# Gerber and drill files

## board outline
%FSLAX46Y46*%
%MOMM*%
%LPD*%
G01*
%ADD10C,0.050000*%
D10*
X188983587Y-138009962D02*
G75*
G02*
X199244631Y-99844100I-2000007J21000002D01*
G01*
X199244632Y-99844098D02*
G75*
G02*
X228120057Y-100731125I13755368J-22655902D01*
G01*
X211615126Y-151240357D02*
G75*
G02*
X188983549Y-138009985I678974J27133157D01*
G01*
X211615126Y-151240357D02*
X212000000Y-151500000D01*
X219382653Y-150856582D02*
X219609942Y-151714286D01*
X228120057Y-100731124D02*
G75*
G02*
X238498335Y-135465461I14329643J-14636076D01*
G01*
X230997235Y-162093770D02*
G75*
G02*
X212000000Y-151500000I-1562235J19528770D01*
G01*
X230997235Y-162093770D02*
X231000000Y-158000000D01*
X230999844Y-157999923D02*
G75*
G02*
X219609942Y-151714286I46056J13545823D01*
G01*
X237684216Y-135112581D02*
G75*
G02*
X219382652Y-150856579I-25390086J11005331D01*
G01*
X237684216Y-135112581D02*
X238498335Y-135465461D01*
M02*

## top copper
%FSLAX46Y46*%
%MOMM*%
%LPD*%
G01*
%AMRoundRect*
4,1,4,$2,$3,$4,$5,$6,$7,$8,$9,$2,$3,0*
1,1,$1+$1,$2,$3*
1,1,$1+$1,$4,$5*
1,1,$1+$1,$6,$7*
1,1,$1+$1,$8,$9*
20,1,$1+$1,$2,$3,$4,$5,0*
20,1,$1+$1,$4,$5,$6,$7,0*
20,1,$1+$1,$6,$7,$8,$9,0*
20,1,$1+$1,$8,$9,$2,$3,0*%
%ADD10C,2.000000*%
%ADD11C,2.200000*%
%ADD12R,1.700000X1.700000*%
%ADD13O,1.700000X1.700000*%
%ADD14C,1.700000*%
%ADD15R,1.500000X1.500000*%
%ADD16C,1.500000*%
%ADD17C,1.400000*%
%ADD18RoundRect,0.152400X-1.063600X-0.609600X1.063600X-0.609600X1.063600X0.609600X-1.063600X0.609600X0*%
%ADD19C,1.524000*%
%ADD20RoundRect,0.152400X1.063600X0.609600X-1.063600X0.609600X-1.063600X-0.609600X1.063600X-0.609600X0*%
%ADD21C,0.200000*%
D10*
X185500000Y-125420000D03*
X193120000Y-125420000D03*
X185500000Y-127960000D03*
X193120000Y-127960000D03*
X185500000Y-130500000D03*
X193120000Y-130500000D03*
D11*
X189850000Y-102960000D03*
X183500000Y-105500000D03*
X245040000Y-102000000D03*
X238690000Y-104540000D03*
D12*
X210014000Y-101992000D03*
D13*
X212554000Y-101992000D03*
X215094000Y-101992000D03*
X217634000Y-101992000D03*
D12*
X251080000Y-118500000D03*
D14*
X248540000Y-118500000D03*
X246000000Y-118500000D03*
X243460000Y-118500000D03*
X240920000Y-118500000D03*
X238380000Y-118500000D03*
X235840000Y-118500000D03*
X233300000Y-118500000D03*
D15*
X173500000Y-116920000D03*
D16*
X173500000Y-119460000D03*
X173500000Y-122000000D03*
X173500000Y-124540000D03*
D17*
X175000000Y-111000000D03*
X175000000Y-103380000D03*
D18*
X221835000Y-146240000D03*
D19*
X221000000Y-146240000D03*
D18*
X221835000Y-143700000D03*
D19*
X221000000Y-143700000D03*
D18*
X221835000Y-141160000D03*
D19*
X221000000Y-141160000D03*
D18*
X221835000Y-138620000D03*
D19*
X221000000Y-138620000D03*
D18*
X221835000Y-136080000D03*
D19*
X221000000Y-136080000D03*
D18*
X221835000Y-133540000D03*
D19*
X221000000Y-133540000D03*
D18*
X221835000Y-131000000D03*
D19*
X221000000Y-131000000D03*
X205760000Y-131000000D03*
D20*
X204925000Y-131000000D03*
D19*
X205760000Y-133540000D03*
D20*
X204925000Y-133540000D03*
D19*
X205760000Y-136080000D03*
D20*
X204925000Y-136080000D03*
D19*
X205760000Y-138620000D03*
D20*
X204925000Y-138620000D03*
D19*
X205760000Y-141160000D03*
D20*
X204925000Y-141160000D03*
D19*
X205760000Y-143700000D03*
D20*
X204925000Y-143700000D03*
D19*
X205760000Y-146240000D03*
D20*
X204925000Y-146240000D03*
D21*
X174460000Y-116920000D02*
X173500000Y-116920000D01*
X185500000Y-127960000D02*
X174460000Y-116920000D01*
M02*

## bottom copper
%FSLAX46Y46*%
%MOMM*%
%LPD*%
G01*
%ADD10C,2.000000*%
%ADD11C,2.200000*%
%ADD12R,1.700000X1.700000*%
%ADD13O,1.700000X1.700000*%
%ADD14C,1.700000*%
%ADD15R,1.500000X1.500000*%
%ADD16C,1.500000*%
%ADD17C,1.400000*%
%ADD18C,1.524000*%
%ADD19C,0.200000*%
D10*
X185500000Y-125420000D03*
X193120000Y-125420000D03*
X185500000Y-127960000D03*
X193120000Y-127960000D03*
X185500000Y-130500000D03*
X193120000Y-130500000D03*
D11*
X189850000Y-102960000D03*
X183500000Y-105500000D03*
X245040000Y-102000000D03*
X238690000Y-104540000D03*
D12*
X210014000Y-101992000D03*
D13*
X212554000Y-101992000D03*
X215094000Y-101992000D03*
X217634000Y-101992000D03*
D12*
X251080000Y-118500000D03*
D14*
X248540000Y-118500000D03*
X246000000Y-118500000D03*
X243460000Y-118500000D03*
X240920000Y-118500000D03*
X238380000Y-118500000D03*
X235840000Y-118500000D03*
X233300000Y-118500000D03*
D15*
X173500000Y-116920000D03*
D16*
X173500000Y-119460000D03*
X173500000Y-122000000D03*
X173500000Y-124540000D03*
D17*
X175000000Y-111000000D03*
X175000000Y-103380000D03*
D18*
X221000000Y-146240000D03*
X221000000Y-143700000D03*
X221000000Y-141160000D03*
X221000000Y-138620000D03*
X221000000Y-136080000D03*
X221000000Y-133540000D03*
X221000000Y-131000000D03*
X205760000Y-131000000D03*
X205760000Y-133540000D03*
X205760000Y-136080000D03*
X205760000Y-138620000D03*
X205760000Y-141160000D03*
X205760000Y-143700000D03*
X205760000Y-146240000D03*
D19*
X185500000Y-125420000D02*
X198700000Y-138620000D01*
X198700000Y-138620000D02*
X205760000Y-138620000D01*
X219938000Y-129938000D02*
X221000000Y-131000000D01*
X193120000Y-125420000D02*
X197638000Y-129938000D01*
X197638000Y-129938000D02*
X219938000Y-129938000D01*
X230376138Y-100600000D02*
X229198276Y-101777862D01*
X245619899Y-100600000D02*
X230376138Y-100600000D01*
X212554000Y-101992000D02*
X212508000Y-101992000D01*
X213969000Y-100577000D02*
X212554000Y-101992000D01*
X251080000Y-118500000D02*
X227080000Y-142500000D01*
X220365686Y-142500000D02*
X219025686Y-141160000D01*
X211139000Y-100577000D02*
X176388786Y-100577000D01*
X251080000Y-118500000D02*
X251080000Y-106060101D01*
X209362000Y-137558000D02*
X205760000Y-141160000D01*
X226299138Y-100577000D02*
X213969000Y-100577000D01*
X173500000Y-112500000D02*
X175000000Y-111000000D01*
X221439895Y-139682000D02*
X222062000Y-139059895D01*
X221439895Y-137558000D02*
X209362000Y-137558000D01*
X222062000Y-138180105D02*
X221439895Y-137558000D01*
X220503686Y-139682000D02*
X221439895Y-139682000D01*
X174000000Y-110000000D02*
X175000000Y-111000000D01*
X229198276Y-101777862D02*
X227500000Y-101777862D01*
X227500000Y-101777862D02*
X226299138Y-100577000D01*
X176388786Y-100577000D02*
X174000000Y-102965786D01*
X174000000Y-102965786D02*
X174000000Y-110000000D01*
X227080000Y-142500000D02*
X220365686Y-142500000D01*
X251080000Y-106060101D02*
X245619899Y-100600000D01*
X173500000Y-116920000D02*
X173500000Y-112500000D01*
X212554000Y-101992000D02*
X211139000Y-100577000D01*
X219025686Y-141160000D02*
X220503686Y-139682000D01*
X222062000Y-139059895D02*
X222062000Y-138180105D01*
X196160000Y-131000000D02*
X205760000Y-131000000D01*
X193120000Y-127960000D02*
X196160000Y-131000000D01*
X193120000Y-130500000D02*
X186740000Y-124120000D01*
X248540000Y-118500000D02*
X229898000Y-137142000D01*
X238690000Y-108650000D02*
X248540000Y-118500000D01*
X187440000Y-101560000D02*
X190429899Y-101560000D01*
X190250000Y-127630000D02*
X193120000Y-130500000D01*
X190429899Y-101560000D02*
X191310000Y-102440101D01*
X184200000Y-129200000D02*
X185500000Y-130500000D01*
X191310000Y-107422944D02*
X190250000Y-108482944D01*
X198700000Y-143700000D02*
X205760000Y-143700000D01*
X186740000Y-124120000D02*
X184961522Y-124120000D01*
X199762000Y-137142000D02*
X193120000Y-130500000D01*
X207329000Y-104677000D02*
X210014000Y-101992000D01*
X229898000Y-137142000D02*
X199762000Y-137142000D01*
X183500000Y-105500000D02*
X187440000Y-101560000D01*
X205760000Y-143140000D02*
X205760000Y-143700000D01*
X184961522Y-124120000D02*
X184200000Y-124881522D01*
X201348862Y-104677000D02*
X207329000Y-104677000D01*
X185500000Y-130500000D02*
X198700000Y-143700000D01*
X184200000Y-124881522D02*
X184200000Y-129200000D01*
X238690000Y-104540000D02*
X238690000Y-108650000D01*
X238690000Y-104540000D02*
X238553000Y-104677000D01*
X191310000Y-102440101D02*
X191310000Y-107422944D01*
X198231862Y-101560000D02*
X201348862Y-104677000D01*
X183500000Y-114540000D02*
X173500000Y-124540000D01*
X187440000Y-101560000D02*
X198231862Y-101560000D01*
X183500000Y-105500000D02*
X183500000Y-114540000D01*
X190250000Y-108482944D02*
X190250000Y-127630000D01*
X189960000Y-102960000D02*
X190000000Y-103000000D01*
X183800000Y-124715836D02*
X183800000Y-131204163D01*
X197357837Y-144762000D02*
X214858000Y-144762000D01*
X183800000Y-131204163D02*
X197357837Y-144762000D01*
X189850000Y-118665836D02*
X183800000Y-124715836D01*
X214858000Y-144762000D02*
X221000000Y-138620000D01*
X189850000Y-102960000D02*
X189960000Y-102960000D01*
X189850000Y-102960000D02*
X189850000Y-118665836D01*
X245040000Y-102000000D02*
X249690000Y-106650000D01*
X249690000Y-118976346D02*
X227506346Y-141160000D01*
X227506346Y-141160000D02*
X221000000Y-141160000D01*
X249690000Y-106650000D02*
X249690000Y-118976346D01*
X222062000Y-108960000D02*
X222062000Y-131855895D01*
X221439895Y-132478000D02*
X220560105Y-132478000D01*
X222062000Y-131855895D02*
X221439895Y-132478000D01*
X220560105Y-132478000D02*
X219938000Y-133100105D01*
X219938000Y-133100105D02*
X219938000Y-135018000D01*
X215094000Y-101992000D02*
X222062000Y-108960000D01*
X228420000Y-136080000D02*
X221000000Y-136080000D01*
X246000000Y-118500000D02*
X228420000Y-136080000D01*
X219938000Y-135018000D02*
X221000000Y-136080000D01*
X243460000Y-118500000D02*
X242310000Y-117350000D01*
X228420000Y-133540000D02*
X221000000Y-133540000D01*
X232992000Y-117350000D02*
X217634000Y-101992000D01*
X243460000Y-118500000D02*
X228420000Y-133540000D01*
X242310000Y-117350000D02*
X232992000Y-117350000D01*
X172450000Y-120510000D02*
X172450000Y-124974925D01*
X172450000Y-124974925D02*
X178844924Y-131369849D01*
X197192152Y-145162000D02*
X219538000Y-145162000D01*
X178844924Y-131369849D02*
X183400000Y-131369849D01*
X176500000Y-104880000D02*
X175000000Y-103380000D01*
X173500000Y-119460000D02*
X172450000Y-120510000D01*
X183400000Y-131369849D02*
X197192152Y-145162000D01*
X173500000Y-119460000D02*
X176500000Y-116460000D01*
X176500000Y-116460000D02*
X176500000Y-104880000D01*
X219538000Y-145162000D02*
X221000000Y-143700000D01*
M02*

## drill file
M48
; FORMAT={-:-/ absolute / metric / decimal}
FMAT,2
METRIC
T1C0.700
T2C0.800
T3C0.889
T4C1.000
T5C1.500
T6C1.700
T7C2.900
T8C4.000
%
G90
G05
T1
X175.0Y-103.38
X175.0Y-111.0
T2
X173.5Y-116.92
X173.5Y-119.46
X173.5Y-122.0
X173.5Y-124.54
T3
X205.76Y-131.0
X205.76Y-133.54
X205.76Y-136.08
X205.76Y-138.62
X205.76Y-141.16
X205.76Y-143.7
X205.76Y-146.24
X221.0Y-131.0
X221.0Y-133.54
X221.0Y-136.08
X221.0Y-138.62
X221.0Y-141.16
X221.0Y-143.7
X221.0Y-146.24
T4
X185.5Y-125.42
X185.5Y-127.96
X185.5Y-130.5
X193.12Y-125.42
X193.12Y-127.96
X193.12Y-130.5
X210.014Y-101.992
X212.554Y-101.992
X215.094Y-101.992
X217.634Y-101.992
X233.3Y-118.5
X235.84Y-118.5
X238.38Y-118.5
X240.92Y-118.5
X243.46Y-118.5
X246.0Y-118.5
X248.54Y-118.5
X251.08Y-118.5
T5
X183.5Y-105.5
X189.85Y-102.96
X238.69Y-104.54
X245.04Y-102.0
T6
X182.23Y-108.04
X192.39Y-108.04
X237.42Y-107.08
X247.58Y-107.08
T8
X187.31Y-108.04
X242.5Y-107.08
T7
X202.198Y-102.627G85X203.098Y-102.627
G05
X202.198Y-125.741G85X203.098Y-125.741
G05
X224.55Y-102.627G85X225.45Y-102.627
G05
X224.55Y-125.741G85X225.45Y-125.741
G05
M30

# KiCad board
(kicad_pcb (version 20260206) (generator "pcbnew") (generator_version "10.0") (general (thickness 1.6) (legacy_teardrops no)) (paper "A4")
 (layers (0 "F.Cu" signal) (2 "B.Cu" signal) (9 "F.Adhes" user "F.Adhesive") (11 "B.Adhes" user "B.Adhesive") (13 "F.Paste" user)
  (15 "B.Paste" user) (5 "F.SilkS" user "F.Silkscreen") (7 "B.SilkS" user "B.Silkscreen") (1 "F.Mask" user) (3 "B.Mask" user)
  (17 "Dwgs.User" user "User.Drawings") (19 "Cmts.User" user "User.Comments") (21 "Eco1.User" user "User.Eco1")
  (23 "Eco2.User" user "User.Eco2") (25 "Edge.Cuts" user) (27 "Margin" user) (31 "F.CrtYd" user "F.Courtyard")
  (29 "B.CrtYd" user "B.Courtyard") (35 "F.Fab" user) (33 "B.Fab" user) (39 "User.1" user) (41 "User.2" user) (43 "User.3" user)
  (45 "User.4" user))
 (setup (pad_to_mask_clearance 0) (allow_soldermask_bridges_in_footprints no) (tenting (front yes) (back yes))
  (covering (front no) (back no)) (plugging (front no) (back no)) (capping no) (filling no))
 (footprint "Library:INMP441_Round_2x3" (layer "F.Cu") (at 185.5 125.42)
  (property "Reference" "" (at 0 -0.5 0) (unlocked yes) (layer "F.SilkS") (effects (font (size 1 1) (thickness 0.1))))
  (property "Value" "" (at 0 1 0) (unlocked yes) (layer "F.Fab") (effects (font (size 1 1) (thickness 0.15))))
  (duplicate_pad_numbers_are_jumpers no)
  (pad "1" thru_hole circle (at 0 0) (size 2 2) (drill 1) (layers "*.Cu" "*.Mask") (remove_unused_layers no) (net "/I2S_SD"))
  (pad "2" thru_hole circle (at 7.62 0) (size 2 2) (drill 1) (layers "*.Cu" "*.Mask") (remove_unused_layers no) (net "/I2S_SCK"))
  (pad "3" thru_hole circle (at 0 2.54) (size 2 2) (drill 1) (layers "*.Cu" "*.Mask") (remove_unused_layers no) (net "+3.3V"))
  (pad "4" thru_hole circle (at 7.62 2.54) (size 2 2) (drill 1) (layers "*.Cu" "*.Mask") (remove_unused_layers no) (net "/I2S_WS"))
  (pad "5" thru_hole circle (at 0 5.08) (size 2 2) (drill 1) (layers "*.Cu" "*.Mask") (remove_unused_layers no) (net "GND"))
  (pad "6" thru_hole circle (at 7.62 5.08) (size 2 2) (drill 1) (layers "*.Cu" "*.Mask") (remove_unused_layers no) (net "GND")))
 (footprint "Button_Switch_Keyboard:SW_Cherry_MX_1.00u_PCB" (layer "F.Cu") (at 189.85 102.96)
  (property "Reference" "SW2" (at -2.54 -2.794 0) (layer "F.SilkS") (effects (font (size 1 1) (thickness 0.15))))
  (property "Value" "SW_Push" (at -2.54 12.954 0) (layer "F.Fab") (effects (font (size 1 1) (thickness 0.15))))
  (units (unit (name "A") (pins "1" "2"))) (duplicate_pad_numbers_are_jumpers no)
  (pad "" np_thru_hole circle (at -7.62 5.08) (size 1.7 1.7) (drill 1.7) (layers "*.Cu" "*.Mask"))
  (pad "" np_thru_hole circle (at -2.54 5.08) (size 4 4) (drill 4) (layers "*.Cu" "*.Mask"))
  (pad "" np_thru_hole circle (at 2.54 5.08) (size 1.7 1.7) (drill 1.7) (layers "*.Cu" "*.Mask"))
  (pad "1" thru_hole circle (at 0 0) (size 2.2 2.2) (drill 1.5) (layers "*.Cu" "*.Mask") (remove_unused_layers no) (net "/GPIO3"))
  (pad "2" thru_hole circle (at -6.35 2.54) (size 2.2 2.2) (drill 1.5) (layers "*.Cu" "*.Mask") (remove_unused_layers no) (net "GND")))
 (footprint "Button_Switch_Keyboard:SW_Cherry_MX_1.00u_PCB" (layer "F.Cu") (at 245.04 102)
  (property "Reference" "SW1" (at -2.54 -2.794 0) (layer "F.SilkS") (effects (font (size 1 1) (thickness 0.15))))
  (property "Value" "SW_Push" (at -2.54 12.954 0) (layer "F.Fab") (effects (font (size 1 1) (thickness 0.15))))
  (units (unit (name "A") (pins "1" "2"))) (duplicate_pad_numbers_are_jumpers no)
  (pad "" np_thru_hole circle (at -7.62 5.08) (size 1.7 1.7) (drill 1.7) (layers "*.Cu" "*.Mask"))
  (pad "" np_thru_hole circle (at -2.54 5.08) (size 4 4) (drill 4) (layers "*.Cu" "*.Mask"))
  (pad "" np_thru_hole circle (at 2.54 5.08) (size 1.7 1.7) (drill 1.7) (layers "*.Cu" "*.Mask"))
  (pad "1" thru_hole circle (at 0 0) (size 2.2 2.2) (drill 1.5) (layers "*.Cu" "*.Mask") (remove_unused_layers no) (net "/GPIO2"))
  (pad "2" thru_hole circle (at -6.35 2.54) (size 2.2 2.2) (drill 1.5) (layers "*.Cu" "*.Mask") (remove_unused_layers no) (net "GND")))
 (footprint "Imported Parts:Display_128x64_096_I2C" (layer "F.Cu") (at 213.824 101.992)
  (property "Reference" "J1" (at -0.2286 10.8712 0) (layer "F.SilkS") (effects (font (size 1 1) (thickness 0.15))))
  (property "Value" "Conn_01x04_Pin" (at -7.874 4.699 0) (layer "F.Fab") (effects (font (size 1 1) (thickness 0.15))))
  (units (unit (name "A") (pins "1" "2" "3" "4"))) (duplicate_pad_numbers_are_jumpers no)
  (pad "" np_thru_hole oval (at -11.176 0.635) (size 3.8 2.9) (drill oval 3.8 2.9) (layers "*.Cu" "*.Mask"))
  (pad "" np_thru_hole oval (at -11.176 23.749) (size 3.8 2.9) (drill oval 3.8 2.9) (layers "*.Cu" "*.Mask"))
  (pad "" np_thru_hole oval (at 11.176 0.635) (size 3.8 2.9) (drill oval 3.8 2.9) (layers "*.Cu" "*.Mask"))
  (pad "" np_thru_hole oval (at 11.176 23.749) (size 3.8 2.9) (drill oval 3.8 2.9) (layers "*.Cu" "*.Mask"))
  (pad "1" thru_hole rect (at -3.81 0 90) (size 1.7 1.7) (drill 1) (layers "*.Cu" "*.Mask") (remove_unused_layers no) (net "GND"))
  (pad "2" thru_hole oval (at -1.27 0 90) (size 1.7 1.7) (drill 1) (layers "*.Cu" "*.Mask") (remove_unused_layers no) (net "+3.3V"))
  (pad "3" thru_hole oval (at 1.27 0 90) (size 1.7 1.7) (drill 1) (layers "*.Cu" "*.Mask") (remove_unused_layers no) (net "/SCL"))
  (pad "4" thru_hole oval (at 3.81 0 90) (size 1.7 1.7) (drill 1) (layers "*.Cu" "*.Mask") (remove_unused_layers no) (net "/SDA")))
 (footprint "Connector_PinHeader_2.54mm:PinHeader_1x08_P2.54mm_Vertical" (layer "F.Cu") (at 251.08 118.5 -90)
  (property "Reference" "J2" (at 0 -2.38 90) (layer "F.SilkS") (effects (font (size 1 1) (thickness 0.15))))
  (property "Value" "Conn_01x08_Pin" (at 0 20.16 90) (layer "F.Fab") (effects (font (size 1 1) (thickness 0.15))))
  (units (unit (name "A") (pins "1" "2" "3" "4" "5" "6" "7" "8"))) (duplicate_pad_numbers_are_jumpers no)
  (pad "1" thru_hole rect (at 0 0 270) (size 1.7 1.7) (drill 1) (layers "*.Cu" "*.Mask") (remove_unused_layers no) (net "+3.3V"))
  (pad "2" thru_hole circle (at 0 2.54 270) (size 1.7 1.7) (drill 1) (layers "*.Cu" "*.Mask") (remove_unused_layers no) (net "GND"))
  (pad "3" thru_hole circle (at 0 5.08 270) (size 1.7 1.7) (drill 1) (layers "*.Cu" "*.Mask") (remove_unused_layers no) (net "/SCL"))
  (pad "4" thru_hole circle (at 0 7.62 270) (size 1.7 1.7) (drill 1) (layers "*.Cu" "*.Mask") (remove_unused_layers no) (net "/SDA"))
  (pad "5" thru_hole circle (at 0 10.16 270) (size 1.7 1.7) (drill 1) (layers "*.Cu" "*.Mask") (remove_unused_layers no)
   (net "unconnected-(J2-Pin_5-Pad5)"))
  (pad "6" thru_hole circle (at 0 12.7 270) (size 1.7 1.7) (drill 1) (layers "*.Cu" "*.Mask") (remove_unused_layers no)
   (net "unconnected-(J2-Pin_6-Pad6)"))
  (pad "7" thru_hole circle (at 0 15.24 270) (size 1.7 1.7) (drill 1) (layers "*.Cu" "*.Mask") (remove_unused_layers no)
   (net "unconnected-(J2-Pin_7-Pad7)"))
  (pad "8" thru_hole circle (at 0 17.78 270) (size 1.7 1.7) (drill 1) (layers "*.Cu" "*.Mask") (remove_unused_layers no)
   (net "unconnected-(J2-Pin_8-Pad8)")))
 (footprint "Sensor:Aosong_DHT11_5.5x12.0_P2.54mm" (layer "F.Cu") (at 173.5 116.92)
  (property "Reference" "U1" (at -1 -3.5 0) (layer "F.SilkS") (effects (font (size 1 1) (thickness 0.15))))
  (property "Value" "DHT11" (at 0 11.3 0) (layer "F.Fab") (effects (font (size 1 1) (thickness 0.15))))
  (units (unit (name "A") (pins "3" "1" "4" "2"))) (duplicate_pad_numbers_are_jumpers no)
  (pad "1" thru_hole rect (at 0 0) (size 1.5 1.5) (drill 0.8) (layers "*.Cu" "*.Mask") (remove_unused_layers no) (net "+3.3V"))
  (pad "2" thru_hole circle (at 0 2.54) (size 1.5 1.5) (drill 0.8) (layers "*.Cu" "*.Mask") (remove_unused_layers no) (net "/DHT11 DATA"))
  (pad "3" thru_hole circle (at 0 5.08) (size 1.5 1.5) (drill 0.8) (layers "*.Cu" "*.Mask") (remove_unused_layers no)
   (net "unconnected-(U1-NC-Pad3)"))
  (pad "4" thru_hole circle (at 0 7.62) (size 1.5 1.5) (drill 0.8) (layers "*.Cu" "*.Mask") (remove_unused_layers no) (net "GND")))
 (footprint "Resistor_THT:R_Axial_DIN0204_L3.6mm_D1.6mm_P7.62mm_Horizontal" (layer "F.Cu") (at 175 111 90)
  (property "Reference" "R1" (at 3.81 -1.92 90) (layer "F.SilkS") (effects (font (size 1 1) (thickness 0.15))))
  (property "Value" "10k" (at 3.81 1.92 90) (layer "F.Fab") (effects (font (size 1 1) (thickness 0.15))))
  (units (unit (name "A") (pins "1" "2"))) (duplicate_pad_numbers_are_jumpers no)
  (pad "1" thru_hole circle (at 0 0 90) (size 1.4 1.4) (drill 0.7) (layers "*.Cu" "*.Mask") (remove_unused_layers no) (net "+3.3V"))
  (pad "2" thru_hole circle (at 7.62 0 90) (size 1.4 1.4) (drill 0.7) (layers "*.Cu" "*.Mask") (remove_unused_layers no) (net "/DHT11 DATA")))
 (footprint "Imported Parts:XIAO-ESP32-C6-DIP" (layer "F.Cu") (at 213.38 138.62 -90)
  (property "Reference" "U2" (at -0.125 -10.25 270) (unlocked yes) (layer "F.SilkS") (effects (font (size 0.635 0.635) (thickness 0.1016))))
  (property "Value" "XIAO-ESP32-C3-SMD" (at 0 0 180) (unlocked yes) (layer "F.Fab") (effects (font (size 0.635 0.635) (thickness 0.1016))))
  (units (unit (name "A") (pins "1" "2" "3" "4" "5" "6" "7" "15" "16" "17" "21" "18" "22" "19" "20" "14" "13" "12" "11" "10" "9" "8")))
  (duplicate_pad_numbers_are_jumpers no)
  (pad "1" smd roundrect (at 7.62 -8.455) (size 2.432 1.524) (layers "F.Cu" "F.Mask") (roundrect_rratio 0.1)
   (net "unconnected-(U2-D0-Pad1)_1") (thermal_bridge_angle 45))
  (pad "1" thru_hole circle (at 7.62 -7.62) (size 1.524 1.524) (drill 0.889) (layers "*.Cu" "*.Mask") (remove_unused_layers no)
   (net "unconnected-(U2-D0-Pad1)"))
  (pad "2" smd roundrect (at 5.08 -8.455) (size 2.432 1.524) (layers "F.Cu" "F.Mask") (roundrect_rratio 0.1) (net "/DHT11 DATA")
   (thermal_bridge_angle 45))
  (pad "2" thru_hole circle (at 5.08 -7.62) (size 1.524 1.524) (drill 0.889) (layers "*.Cu" "*.Mask") (remove_unused_layers no)
   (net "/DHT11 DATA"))
  (pad "3" smd roundrect (at 2.54 -8.455) (size 2.432 1.524) (layers "F.Cu" "F.Mask") (roundrect_rratio 0.1) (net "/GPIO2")
   (thermal_bridge_angle 45))
  (pad "3" thru_hole circle (at 2.54 -7.62) (size 1.524 1.524) (drill 0.889) (layers "*.Cu" "*.Mask") (remove_unused_layers no)
   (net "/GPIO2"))
  (pad "4" smd roundrect (at 0 -8.455) (size 2.432 1.524) (layers "F.Cu" "F.Mask") (roundrect_rratio 0.1) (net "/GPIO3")
   (thermal_bridge_angle 45))
  (pad "4" thru_hole circle (at 0 -7.62) (size 1.524 1.524) (drill 0.889) (layers "*.Cu" "*.Mask") (remove_unused_layers no) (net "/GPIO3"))
  (pad "5" smd roundrect (at -2.54 -8.455) (size 2.432 1.524) (layers "F.Cu" "F.Mask") (roundrect_rratio 0.1) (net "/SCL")
   (thermal_bridge_angle 45))
  (pad "5" thru_hole circle (at -2.54 -7.62) (size 1.524 1.524) (drill 0.889) (layers "*.Cu" "*.Mask") (remove_unused_layers no)
   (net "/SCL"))
  (pad "6" smd roundrect (at -5.08 -8.455) (size 2.432 1.524) (layers "F.Cu" "F.Mask") (roundrect_rratio 0.1) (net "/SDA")
   (thermal_bridge_angle 45))
  (pad "6" thru_hole circle (at -5.08 -7.62) (size 1.524 1.524) (drill 0.889) (layers "*.Cu" "*.Mask") (remove_unused_layers no)
   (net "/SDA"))
  (pad "7" smd roundrect (at -7.62 -8.455) (size 2.432 1.524) (layers "F.Cu" "F.Mask") (roundrect_rratio 0.1) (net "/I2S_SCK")
   (thermal_bridge_angle 45))
  (pad "7" thru_hole circle (at -7.62 -7.62) (size 1.524 1.524) (drill 0.889) (layers "*.Cu" "*.Mask") (remove_unused_layers no)
   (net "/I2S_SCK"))
  (pad "8" thru_hole circle (at -7.62 7.62 180) (size 1.524 1.524) (drill 0.889) (layers "*.Cu" "*.Mask") (remove_unused_layers no)
   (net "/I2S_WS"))
  (pad "8" smd roundrect (at -7.62 8.455 180) (size 2.432 1.524) (layers "F.Cu" "F.Mask") (roundrect_rratio 0.1) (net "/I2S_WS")
   (thermal_bridge_angle 45))
  (pad "9" thru_hole circle (at -5.08 7.62 180) (size 1.524 1.524) (drill 0.889) (layers "*.Cu" "*.Mask") (remove_unused_layers no)
   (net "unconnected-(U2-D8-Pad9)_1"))
  (pad "9" smd roundrect (at -5.08 8.455 180) (size 2.432 1.524) (layers "F.Cu" "F.Mask") (roundrect_rratio 0.1)
   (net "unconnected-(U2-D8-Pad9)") (thermal_bridge_angle 45))
  (pad "10" thru_hole circle (at -2.54 7.62 180) (size 1.524 1.524) (drill 0.889) (layers "*.Cu" "*.Mask") (remove_unused_layers no)
   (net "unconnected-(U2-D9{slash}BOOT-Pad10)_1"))
  (pad "10" smd roundrect (at -2.54 8.455 180) (size 2.432 1.524) (layers "F.Cu" "F.Mask") (roundrect_rratio 0.1)
   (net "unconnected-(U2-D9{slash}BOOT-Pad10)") (thermal_bridge_angle 45))
  (pad "11" thru_hole circle (at 0 7.62 180) (size 1.524 1.524) (drill 0.889) (layers "*.Cu" "*.Mask") (remove_unused_layers no)
   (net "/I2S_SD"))
  (pad "11" smd roundrect (at 0 8.455 180) (size 2.432 1.524) (layers "F.Cu" "F.Mask") (roundrect_rratio 0.1) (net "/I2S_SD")
   (thermal_bridge_angle 45))
  (pad "12" thru_hole circle (at 2.54 7.62 180) (size 1.524 1.524) (drill 0.889) (layers "*.Cu" "*.Mask") (remove_unused_layers no)
   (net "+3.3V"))
  (pad "12" smd roundrect (at 2.54 8.455 180) (size 2.432 1.524) (layers "F.Cu" "F.Mask") (roundrect_rratio 0.1) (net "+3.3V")
   (thermal_bridge_angle 45))
  (pad "13" thru_hole circle (at 5.08 7.62 180) (size 1.524 1.524) (drill 0.889) (layers "*.Cu" "*.Mask") (remove_unused_layers no)
   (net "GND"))
  (pad "13" smd roundrect (at 5.08 8.455 180) (size 2.432 1.524) (layers "F.Cu" "F.Mask") (roundrect_rratio 0.1) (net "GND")
   (thermal_bridge_angle 45))
  (pad "14" thru_hole circle (at 7.62 7.62 180) (size 1.524 1.524) (drill 0.889) (layers "*.Cu" "*.Mask") (remove_unused_layers no)
   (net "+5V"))
  (pad "14" smd roundrect (at 7.62 8.455 180) (size 2.432 1.524) (layers "F.Cu" "F.Mask") (roundrect_rratio 0.1) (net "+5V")
   (thermal_bridge_angle 45)))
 (gr_arc (start 188.983587 138.009962) (mid 166.611969 111.532968) (end 199.244633 99.844097) (stroke (width 0.05) (type default))
  (layer "Edge.Cuts"))
 (gr_arc (start 199.244632 99.844098) (mid 213.813817 96.00778) (end 228.120057 100.731125) (stroke (width 0.05) (type default))
  (layer "Edge.Cuts"))
 (gr_arc (start 211.615126 151.240357) (mid 198.596121 147.538665) (end 188.983587 138.009962) (stroke (width 0.05) (type default))
  (layer "Edge.Cuts"))
 (gr_line (start 211.615126 151.240357) (end 212 151.5) (stroke (width 0.05) (type default)) (layer "Edge.Cuts"))
 (gr_line (start 219.382653 150.856582) (end 219.609942 151.714286) (stroke (width 0.05) (type default)) (layer "Edge.Cuts"))
 (gr_arc (start 228.120057 100.731124) (mid 262.075381 109.50324) (end 238.498335 135.465461) (stroke (width 0.05) (type default))
  (layer "Edge.Cuts"))
 (gr_arc (start 230.997235 162.09377) (mid 219.893346 159.675531) (end 212 151.5) (stroke (width 0.05) (type default)) (layer "Edge.Cuts"))
 (gr_line (start 230.997235 162.09377) (end 231 158) (stroke (width 0.05) (type default)) (layer "Edge.Cuts"))
 (gr_arc (start 230.999844 157.999923) (mid 224.500942 156.313905) (end 219.609942 151.714286) (stroke (width 0.05) (type default))
  (layer "Edge.Cuts"))
 (gr_arc (start 237.684216 135.112581) (mid 230.34083 145.085583) (end 219.382653 150.856582) (stroke (width 0.05) (type default))
  (layer "Edge.Cuts"))
 (gr_line (start 237.684216 135.112581) (end 238.498335 135.465461) (stroke (width 0.05) (type default)) (layer "Edge.Cuts"))
 (segment (start 185.5 125.42) (end 198.7 138.62) (width 0.2) (layer "B.Cu") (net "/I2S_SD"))
 (segment (start 198.7 138.62) (end 205.76 138.62) (width 0.2) (layer "B.Cu") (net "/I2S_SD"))
 (segment (start 219.938 129.938) (end 221 131) (width 0.2) (layer "B.Cu") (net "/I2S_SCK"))
 (segment (start 193.12 125.42) (end 197.638 129.938) (width 0.2) (layer "B.Cu") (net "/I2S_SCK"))
 (segment (start 197.638 129.938) (end 219.938 129.938) (width 0.2) (layer "B.Cu") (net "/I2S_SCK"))
 (segment (start 174.46 116.92) (end 173.5 116.92) (width 0.2) (layer "F.Cu") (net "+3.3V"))
 (segment (start 185.5 127.96) (end 174.46 116.92) (width 0.2) (layer "F.Cu") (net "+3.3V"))
 (segment (start 230.376138 100.6) (end 229.198276 101.777862) (width 0.2) (layer "B.Cu") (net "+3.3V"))
 (segment (start 245.619899 100.6) (end 230.376138 100.6) (width 0.2) (layer "B.Cu") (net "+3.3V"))
 (segment (start 212.554 101.992) (end 212.508 101.992) (width 0.2) (layer "B.Cu") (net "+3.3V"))
 (segment (start 213.969 100.577) (end 212.554 101.992) (width 0.2) (layer "B.Cu") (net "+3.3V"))
 (segment (start 251.08 118.5) (end 227.08 142.5) (width 0.2) (layer "B.Cu") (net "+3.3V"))
 (segment (start 220.365686 142.5) (end 219.025686 141.16) (width 0.2) (layer "B.Cu") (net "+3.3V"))
 (segment (start 211.139 100.577) (end 176.388786 100.577) (width 0.2) (layer "B.Cu") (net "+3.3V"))
 (segment (start 251.08 118.5) (end 251.08 106.060101) (width 0.2) (layer "B.Cu") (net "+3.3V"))
 (segment (start 209.362 137.558) (end 205.76 141.16) (width 0.2) (layer "B.Cu") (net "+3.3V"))
 (segment (start 226.299138 100.577) (end 213.969 100.577) (width 0.2) (layer "B.Cu") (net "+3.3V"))
 (segment (start 173.5 112.5) (end 175 111) (width 0.2) (layer "B.Cu") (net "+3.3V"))
 (segment (start 221.439895 139.682) (end 222.062 139.059895) (width 0.2) (layer "B.Cu") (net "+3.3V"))
 (segment (start 221.439895 137.558) (end 209.362 137.558) (width 0.2) (layer "B.Cu") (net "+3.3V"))
 (segment (start 222.062 138.180105) (end 221.439895 137.558) (width 0.2) (layer "B.Cu") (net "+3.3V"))
 (segment (start 220.503686 139.682) (end 221.439895 139.682) (width 0.2) (layer "B.Cu") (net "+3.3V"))
 (segment (start 174 110) (end 175 111) (width 0.2) (layer "B.Cu") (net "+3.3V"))
 (segment (start 229.198276 101.777862) (end 227.5 101.777862) (width 0.2) (layer "B.Cu") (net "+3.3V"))
 (segment (start 227.5 101.777862) (end 226.299138 100.577) (width 0.2) (layer "B.Cu") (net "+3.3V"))
 (segment (start 176.388786 100.577) (end 174 102.965786) (width 0.2) (layer "B.Cu") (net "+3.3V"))
 (segment (start 174 102.965786) (end 174 110) (width 0.2) (layer "B.Cu") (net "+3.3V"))
 (segment (start 227.08 142.5) (end 220.365686 142.5) (width 0.2) (layer "B.Cu") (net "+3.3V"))
 (segment (start 251.08 106.060101) (end 245.619899 100.6) (width 0.2) (layer "B.Cu") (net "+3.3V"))
 (segment (start 173.5 116.92) (end 173.5 112.5) (width 0.2) (layer "B.Cu") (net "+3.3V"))
 (segment (start 212.554 101.992) (end 211.139 100.577) (width 0.2) (layer "B.Cu") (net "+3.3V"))
 (segment (start 219.025686 141.16) (end 220.503686 139.682) (width 0.2) (layer "B.Cu") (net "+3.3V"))
 (segment (start 222.062 139.059895) (end 222.062 138.180105) (width 0.2) (layer "B.Cu") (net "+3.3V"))
 (segment (start 196.16 131) (end 205.76 131) (width 0.2) (layer "B.Cu") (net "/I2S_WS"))
 (segment (start 193.12 127.96) (end 196.16 131) (width 0.2) (layer "B.Cu") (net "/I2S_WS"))
 (segment (start 193.12 130.5) (end 186.74 124.12) (width 0.2) (layer "B.Cu") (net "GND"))
 (segment (start 248.54 118.5) (end 229.898 137.142) (width 0.2) (layer "B.Cu") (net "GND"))
 (segment (start 238.69 108.65) (end 248.54 118.5) (width 0.2) (layer "B.Cu") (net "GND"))
 (segment (start 187.44 101.56) (end 190.429899 101.56) (width 0.2) (layer "B.Cu") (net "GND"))
 (segment (start 190.25 127.63) (end 193.12 130.5) (width 0.2) (layer "B.Cu") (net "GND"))
 (segment (start 190.429899 101.56) (end 191.31 102.440101) (width 0.2) (layer "B.Cu") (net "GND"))
 (segment (start 184.2 129.2) (end 185.5 130.5) (width 0.2) (layer "B.Cu") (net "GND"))
 (segment (start 191.31 107.422944) (end 190.25 108.482944) (width 0.2) (layer "B.Cu") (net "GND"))
 (segment (start 198.7 143.7) (end 205.76 143.7) (width 0.2) (layer "B.Cu") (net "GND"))
 (segment (start 186.74 124.12) (end 184.961522 124.12) (width 0.2) (layer "B.Cu") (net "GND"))
 (segment (start 199.762 137.142) (end 193.12 130.5) (width 0.2) (layer "B.Cu") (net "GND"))
 (segment (start 207.329 104.677) (end 210.014 101.992) (width 0.2) (layer "B.Cu") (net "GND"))
 (segment (start 229.898 137.142) (end 199.762 137.142) (width 0.2) (layer "B.Cu") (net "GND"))
 (segment (start 183.5 105.5) (end 187.44 101.56) (width 0.2) (layer "B.Cu") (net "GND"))
 (segment (start 205.76 143.14) (end 205.76 143.7) (width 0.2) (layer "B.Cu") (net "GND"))
 (segment (start 184.961522 124.12) (end 184.2 124.881522) (width 0.2) (layer "B.Cu") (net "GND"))
 (segment (start 201.348862 104.677) (end 207.329 104.677) (width 0.2) (layer "B.Cu") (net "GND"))
 (segment (start 185.5 130.5) (end 198.7 143.7) (width 0.2) (layer "B.Cu") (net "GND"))
 (segment (start 184.2 124.881522) (end 184.2 129.2) (width 0.2) (layer "B.Cu") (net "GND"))
 (segment (start 238.69 104.54) (end 238.69 108.65) (width 0.2) (layer "B.Cu") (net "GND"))
 (segment (start 238.69 104.54) (end 238.553 104.677) (width 0.2) (layer "B.Cu") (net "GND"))
 (segment (start 191.31 102.440101) (end 191.31 107.422944) (width 0.2) (layer "B.Cu") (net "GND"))
 (segment (start 198.231862 101.56) (end 201.348862 104.677) (width 0.2) (layer "B.Cu") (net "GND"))
 (segment (start 183.5 114.54) (end 173.5 124.54) (width 0.2) (layer "B.Cu") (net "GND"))
 (segment (start 187.44 101.56) (end 198.231862 101.56) (width 0.2) (layer "B.Cu") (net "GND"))
 (segment (start 183.5 105.5) (end 183.5 114.54) (width 0.2) (layer "B.Cu") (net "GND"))
 (segment (start 190.25 108.482944) (end 190.25 127.63) (width 0.2) (layer "B.Cu") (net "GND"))
 (segment (start 189.96 102.96) (end 190 103) (width 0.2) (layer "B.Cu") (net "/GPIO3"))
 (segment (start 183.8 124.715836) (end 183.8 131.204163) (width 0.2) (layer "B.Cu") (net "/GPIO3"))
 (segment (start 197.357837 144.762) (end 214.858 144.762) (width 0.2) (layer "B.Cu") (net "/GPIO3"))
 (segment (start 183.8 131.204163) (end 197.357837 144.762) (width 0.2) (layer "B.Cu") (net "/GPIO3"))
 (segment (start 189.85 118.665836) (end 183.8 124.715836) (width 0.2) (layer "B.Cu") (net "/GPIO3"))
 (segment (start 214.858 144.762) (end 221 138.62) (width 0.2) (layer "B.Cu") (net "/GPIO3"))
 (segment (start 189.85 102.96) (end 189.96 102.96) (width 0.2) (layer "B.Cu") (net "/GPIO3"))
 (segment (start 189.85 102.96) (end 189.85 118.665836) (width 0.2) (layer "B.Cu") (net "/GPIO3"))
 (segment (start 245.04 102) (end 249.69 106.65) (width 0.2) (layer "B.Cu") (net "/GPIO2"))
 (segment (start 249.69 118.976346) (end 227.506346 141.16) (width 0.2) (layer "B.Cu") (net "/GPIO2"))
 (segment (start 227.506346 141.16) (end 221 141.16) (width 0.2) (layer "B.Cu") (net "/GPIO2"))
 (segment (start 249.69 106.65) (end 249.69 118.976346) (width 0.2) (layer "B.Cu") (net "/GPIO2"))
 (segment (start 222.062 108.96) (end 222.062 131.855895) (width 0.2) (layer "B.Cu") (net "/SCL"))
 (segment (start 221.439895 132.478) (end 220.560105 132.478) (width 0.2) (layer "B.Cu") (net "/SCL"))
 (segment (start 222.062 131.855895) (end 221.439895 132.478) (width 0.2) (layer "B.Cu") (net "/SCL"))
 (segment (start 220.560105 132.478) (end 219.938 133.100105) (width 0.2) (layer "B.Cu") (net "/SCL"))
 (segment (start 219.938 133.100105) (end 219.938 135.018) (width 0.2) (layer "B.Cu") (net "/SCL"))
 (segment (start 215.094 101.992) (end 222.062 108.96) (width 0.2) (layer "B.Cu") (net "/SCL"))
 (segment (start 228.42 136.08) (end 221 136.08) (width 0.2) (layer "B.Cu") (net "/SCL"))
 (segment (start 246 118.5) (end 228.42 136.08) (width 0.2) (layer "B.Cu") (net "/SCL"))
 (segment (start 219.938 135.018) (end 221 136.08) (width 0.2) (layer "B.Cu") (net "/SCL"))
 (segment (start 243.46 118.5) (end 242.31 117.35) (width 0.2) (layer "B.Cu") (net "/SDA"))
 (segment (start 228.42 133.54) (end 221 133.54) (width 0.2) (layer "B.Cu") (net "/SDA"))
 (segment (start 232.992 117.35) (end 217.634 101.992) (width 0.2) (layer "B.Cu") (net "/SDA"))
 (segment (start 243.46 118.5) (end 228.42 133.54) (width 0.2) (layer "B.Cu") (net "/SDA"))
 (segment (start 242.31 117.35) (end 232.992 117.35) (width 0.2) (layer "B.Cu") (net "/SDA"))
 (segment (start 172.45 120.51) (end 172.45 124.974925) (width 0.2) (layer "B.Cu") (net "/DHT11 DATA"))
 (segment (start 172.45 124.974925) (end 178.844924 131.369849) (width 0.2) (layer "B.Cu") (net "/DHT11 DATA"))
 (segment (start 197.192152 145.162) (end 219.538 145.162) (width 0.2) (layer "B.Cu") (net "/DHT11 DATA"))
 (segment (start 178.844924 131.369849) (end 183.4 131.369849) (width 0.2) (layer "B.Cu") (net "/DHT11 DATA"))
 (segment (start 176.5 104.88) (end 175 103.38) (width 0.2) (layer "B.Cu") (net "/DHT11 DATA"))
 (segment (start 173.5 119.46) (end 172.45 120.51) (width 0.2) (layer "B.Cu") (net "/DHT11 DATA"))
 (segment (start 183.4 131.369849) (end 197.192152 145.162) (width 0.2) (layer "B.Cu") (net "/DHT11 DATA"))
 (segment (start 173.5 119.46) (end 176.5 116.46) (width 0.2) (layer "B.Cu") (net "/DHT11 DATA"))
 (segment (start 176.5 116.46) (end 176.5 104.88) (width 0.2) (layer "B.Cu") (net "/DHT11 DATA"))
 (segment (start 219.538 145.162) (end 221 143.7) (width 0.2) (layer "B.Cu") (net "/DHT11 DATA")))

